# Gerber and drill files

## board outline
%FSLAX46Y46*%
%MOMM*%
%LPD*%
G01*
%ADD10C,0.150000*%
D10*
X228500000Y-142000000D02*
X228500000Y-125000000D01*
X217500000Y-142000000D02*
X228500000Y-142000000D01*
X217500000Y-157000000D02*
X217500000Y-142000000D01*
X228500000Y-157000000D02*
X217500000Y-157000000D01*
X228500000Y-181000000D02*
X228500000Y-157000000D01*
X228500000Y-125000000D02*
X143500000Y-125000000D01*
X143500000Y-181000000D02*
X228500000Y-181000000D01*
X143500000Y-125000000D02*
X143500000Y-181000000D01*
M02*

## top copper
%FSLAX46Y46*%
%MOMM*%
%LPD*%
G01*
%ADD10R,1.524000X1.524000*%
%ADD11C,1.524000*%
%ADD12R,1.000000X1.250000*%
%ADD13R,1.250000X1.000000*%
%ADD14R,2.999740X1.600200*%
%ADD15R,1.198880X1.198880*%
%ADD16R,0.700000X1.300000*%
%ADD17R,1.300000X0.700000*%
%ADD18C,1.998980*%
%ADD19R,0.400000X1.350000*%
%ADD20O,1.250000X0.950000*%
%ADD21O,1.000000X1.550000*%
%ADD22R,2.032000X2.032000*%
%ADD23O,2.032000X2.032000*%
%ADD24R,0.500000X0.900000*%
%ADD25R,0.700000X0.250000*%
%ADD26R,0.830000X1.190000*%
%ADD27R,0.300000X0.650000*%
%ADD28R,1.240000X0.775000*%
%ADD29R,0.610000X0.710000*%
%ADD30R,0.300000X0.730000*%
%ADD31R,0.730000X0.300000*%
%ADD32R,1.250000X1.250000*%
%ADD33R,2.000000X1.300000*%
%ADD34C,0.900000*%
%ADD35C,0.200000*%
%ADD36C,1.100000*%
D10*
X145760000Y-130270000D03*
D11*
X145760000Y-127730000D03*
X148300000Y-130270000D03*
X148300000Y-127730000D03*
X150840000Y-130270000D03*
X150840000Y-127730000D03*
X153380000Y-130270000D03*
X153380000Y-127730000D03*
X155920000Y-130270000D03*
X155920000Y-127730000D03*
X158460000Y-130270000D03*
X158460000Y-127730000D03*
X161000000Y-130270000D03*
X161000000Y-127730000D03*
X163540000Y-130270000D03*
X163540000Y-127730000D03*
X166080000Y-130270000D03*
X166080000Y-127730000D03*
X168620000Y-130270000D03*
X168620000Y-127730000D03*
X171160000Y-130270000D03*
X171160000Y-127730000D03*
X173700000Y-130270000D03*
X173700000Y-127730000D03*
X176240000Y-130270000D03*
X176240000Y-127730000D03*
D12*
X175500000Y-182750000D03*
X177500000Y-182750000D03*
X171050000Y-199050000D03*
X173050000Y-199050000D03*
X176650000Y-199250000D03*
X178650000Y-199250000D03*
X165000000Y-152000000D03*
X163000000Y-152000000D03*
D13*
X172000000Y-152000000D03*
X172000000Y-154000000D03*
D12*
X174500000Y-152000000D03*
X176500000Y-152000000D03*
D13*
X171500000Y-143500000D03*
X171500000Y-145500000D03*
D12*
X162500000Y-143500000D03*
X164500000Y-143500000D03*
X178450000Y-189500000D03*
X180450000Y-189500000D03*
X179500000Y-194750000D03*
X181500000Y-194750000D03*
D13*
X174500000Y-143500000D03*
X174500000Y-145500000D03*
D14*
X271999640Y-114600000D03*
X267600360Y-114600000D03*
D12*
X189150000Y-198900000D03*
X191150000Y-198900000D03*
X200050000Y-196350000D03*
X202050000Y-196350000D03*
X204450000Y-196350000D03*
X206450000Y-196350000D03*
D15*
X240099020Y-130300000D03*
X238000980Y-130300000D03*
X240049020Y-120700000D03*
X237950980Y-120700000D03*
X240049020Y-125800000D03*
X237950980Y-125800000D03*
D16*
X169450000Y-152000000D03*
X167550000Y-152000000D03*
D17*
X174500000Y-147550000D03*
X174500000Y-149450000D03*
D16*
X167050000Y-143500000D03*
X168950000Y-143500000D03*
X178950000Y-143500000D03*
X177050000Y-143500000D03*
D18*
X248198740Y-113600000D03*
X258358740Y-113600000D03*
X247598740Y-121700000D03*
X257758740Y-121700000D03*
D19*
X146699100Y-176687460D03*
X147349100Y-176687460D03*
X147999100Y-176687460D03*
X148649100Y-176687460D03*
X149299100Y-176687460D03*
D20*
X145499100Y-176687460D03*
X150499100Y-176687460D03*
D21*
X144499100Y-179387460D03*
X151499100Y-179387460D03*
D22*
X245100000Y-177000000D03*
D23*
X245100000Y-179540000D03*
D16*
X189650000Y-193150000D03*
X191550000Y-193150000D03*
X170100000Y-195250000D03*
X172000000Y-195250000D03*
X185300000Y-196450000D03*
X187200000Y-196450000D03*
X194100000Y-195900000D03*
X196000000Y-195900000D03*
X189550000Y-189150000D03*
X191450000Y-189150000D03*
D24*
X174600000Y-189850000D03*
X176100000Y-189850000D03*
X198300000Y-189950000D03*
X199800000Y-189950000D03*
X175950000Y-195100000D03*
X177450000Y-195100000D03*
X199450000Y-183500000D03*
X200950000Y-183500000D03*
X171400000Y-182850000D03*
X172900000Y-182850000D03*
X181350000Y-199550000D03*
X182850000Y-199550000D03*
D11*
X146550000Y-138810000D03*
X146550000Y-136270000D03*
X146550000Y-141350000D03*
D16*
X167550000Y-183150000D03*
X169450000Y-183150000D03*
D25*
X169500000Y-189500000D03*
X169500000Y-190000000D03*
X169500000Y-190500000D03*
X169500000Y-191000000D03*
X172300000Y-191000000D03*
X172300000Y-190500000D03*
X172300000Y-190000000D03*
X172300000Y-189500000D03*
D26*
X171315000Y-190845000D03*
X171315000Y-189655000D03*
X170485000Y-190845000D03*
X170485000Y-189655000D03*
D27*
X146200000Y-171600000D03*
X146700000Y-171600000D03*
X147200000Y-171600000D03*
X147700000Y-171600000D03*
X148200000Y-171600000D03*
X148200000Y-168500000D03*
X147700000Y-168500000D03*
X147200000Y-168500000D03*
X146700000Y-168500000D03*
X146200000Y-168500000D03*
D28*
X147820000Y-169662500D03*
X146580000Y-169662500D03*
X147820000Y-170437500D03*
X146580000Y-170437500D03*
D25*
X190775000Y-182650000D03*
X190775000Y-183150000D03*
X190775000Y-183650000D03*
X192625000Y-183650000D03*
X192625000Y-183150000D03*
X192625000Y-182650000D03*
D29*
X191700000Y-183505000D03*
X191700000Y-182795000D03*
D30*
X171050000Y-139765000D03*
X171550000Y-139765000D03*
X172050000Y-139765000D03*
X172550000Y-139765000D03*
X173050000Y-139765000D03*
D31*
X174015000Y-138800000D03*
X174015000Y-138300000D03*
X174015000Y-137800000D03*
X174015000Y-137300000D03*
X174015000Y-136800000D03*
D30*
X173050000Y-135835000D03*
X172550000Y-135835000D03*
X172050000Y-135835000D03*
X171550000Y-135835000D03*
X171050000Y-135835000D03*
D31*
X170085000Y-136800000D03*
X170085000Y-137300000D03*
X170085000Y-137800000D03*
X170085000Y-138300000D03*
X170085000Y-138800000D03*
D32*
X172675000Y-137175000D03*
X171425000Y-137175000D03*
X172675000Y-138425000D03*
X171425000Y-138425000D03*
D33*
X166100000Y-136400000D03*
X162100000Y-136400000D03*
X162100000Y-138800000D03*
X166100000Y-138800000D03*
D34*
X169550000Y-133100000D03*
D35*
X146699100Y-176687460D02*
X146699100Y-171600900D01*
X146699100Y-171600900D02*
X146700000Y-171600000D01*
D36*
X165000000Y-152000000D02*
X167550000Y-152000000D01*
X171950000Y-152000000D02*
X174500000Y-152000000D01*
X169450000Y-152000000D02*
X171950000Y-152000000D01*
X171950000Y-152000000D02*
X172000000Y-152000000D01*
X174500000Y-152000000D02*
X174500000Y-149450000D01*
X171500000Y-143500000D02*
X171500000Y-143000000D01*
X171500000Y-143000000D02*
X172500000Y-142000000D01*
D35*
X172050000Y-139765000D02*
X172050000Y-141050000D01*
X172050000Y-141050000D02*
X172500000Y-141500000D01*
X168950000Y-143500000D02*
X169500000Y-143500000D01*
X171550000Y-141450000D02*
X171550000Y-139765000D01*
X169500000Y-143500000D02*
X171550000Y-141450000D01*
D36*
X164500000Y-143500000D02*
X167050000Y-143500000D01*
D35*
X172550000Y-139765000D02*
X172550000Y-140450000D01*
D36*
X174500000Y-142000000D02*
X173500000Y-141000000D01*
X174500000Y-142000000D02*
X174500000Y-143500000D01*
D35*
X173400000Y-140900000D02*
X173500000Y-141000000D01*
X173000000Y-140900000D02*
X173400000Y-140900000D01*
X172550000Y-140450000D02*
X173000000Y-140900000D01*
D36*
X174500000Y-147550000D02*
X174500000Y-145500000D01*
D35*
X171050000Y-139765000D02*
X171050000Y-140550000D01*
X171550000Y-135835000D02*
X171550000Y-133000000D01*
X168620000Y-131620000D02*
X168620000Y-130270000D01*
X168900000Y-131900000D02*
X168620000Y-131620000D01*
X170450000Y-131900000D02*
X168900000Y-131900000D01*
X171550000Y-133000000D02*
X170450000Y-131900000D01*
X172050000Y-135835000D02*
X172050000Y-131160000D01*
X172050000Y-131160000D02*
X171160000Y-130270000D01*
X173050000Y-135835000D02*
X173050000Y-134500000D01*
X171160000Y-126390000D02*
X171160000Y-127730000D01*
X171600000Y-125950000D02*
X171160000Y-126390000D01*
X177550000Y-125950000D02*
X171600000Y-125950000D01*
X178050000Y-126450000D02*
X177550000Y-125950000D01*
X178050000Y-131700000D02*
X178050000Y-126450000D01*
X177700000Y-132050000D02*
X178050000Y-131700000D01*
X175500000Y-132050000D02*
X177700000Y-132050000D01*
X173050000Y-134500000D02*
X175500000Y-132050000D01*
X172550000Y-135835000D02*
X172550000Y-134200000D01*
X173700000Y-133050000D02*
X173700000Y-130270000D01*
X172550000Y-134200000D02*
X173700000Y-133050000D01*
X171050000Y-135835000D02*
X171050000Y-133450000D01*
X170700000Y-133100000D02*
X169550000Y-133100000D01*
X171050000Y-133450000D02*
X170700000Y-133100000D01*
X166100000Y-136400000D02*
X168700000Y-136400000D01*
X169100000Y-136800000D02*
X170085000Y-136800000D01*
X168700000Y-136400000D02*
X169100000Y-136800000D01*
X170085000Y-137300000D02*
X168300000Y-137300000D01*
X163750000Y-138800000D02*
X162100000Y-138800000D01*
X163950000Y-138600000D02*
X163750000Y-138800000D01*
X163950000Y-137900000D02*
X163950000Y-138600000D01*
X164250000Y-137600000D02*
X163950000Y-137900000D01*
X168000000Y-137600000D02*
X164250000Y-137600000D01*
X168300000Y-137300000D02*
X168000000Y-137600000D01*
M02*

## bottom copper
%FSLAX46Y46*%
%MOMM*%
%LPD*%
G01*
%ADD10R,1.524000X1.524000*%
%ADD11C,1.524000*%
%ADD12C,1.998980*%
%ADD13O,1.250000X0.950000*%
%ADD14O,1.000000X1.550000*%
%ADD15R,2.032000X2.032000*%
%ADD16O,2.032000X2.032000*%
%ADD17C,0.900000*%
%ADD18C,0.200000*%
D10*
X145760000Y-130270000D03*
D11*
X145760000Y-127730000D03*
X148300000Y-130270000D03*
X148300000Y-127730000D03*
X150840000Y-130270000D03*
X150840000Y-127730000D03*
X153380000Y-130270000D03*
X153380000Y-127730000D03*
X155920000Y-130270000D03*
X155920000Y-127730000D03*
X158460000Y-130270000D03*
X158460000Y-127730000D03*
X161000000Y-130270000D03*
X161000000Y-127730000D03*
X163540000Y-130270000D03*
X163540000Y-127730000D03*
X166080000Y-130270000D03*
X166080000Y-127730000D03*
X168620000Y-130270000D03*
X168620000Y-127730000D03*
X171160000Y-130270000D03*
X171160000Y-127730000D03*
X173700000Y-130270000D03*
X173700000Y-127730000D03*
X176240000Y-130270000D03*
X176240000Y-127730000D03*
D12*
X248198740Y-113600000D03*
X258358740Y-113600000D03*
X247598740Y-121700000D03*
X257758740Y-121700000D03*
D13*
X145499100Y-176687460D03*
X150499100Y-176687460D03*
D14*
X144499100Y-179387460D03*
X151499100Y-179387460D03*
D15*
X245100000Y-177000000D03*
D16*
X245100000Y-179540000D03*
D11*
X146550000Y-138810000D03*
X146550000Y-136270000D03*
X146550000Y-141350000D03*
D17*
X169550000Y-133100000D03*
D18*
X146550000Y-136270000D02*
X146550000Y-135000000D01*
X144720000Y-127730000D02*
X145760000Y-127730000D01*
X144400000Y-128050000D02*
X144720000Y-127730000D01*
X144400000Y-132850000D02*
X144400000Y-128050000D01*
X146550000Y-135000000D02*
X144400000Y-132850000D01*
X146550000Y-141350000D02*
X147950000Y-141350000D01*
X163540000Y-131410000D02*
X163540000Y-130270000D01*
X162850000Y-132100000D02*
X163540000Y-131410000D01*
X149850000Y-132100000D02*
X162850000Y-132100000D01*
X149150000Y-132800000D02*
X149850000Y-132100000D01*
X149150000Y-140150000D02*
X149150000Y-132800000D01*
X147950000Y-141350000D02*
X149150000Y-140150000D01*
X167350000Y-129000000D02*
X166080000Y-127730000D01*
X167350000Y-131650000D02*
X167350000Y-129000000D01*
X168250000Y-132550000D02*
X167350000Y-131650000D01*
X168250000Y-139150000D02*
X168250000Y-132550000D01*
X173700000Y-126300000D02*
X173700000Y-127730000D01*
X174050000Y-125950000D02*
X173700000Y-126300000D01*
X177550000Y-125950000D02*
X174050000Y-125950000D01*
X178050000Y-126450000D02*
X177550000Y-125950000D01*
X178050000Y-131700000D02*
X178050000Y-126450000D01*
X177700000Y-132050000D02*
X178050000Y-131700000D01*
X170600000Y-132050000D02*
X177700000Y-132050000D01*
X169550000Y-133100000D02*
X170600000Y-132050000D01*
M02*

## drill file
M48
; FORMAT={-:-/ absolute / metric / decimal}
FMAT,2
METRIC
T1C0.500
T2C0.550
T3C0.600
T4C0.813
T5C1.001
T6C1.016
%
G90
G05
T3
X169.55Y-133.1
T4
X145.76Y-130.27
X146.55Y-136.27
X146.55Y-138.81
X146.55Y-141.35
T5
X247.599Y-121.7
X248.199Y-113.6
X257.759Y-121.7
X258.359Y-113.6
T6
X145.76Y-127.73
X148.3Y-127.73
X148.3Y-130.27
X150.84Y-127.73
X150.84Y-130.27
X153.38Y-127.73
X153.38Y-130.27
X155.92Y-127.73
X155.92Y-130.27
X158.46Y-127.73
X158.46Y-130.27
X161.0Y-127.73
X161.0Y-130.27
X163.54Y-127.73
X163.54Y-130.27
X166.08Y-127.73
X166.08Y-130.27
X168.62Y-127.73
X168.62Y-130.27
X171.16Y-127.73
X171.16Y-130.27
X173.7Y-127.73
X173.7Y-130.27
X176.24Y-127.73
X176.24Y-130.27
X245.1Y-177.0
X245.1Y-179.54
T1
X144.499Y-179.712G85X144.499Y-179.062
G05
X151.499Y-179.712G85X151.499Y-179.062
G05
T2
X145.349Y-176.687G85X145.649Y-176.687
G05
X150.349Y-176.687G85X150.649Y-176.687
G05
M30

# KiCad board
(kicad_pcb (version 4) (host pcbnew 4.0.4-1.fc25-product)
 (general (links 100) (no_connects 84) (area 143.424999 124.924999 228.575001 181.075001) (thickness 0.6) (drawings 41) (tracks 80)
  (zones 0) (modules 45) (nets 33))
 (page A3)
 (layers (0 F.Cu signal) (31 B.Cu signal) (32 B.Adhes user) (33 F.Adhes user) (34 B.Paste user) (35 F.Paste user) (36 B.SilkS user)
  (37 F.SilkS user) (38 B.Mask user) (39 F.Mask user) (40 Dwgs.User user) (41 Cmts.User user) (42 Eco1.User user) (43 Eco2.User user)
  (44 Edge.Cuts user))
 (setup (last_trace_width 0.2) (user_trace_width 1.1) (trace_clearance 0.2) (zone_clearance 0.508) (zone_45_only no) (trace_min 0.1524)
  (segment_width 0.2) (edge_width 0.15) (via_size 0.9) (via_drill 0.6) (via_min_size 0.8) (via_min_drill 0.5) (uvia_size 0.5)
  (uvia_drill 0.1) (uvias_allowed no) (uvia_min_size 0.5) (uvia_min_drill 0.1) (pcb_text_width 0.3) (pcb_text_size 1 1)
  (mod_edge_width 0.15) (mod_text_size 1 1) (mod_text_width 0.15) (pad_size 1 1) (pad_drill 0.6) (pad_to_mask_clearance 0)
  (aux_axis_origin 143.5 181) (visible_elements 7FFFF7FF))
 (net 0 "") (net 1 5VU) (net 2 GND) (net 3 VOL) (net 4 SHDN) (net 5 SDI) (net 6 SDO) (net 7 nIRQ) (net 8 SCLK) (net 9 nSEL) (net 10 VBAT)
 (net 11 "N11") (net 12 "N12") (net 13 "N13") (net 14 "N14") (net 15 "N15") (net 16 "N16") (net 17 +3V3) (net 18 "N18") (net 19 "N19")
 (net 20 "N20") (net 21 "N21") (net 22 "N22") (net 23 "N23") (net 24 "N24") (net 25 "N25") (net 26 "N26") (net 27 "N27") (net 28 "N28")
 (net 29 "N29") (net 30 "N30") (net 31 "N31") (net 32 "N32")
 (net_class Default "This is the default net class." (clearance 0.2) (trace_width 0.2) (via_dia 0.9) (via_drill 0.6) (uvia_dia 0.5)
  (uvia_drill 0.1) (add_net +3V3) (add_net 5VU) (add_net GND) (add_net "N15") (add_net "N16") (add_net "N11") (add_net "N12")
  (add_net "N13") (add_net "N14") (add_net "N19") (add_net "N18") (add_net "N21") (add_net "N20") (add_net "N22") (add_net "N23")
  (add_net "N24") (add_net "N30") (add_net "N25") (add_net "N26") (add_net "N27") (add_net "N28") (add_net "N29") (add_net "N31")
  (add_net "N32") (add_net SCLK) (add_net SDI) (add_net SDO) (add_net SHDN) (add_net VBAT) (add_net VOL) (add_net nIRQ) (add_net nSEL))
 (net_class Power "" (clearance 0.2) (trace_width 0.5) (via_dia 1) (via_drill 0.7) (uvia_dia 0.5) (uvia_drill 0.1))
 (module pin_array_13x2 (layer F.Cu) (at 161 129)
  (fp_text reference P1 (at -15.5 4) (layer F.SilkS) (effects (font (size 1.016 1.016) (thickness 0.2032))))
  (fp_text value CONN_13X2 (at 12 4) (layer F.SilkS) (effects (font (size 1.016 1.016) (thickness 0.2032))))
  (pad 1 thru_hole rect (at -15.24 1.27) (size 1.524 1.524) (drill 0.8128) (layers *.Cu *.Mask F.SilkS))
  (pad 2 thru_hole circle (at -15.24 -1.27) (size 1.524 1.524) (drill 1.016) (layers *.Cu *.Mask F.SilkS) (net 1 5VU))
  (pad 3 thru_hole circle (at -12.7 1.27) (size 1.524 1.524) (drill 1.016) (layers *.Cu *.Mask F.SilkS))
  (pad 4 thru_hole circle (at -12.7 -1.27) (size 1.524 1.524) (drill 1.016) (layers *.Cu *.Mask F.SilkS))
  (pad 5 thru_hole circle (at -10.16 1.27) (size 1.524 1.524) (drill 1.016) (layers *.Cu *.Mask F.SilkS))
  (pad 6 thru_hole circle (at -10.16 -1.27) (size 1.524 1.524) (drill 1.016) (layers *.Cu *.Mask F.SilkS) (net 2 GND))
  (pad 7 thru_hole circle (at -7.62 1.27) (size 1.524 1.524) (drill 1.016) (layers *.Cu *.Mask F.SilkS))
  (pad 8 thru_hole circle (at -7.62 -1.27) (size 1.524 1.524) (drill 1.016) (layers *.Cu *.Mask F.SilkS))
  (pad 9 thru_hole circle (at -5.08 1.27) (size 1.524 1.524) (drill 1.016) (layers *.Cu *.Mask F.SilkS))
  (pad 10 thru_hole circle (at -5.08 -1.27) (size 1.524 1.524) (drill 1.016) (layers *.Cu *.Mask F.SilkS))
  (pad 11 thru_hole circle (at -2.54 1.27) (size 1.524 1.524) (drill 1.016) (layers *.Cu *.Mask F.SilkS))
  (pad 12 thru_hole circle (at -2.54 -1.27) (size 1.524 1.524) (drill 1.016) (layers *.Cu *.Mask F.SilkS))
  (pad 13 thru_hole circle (at 0 1.27) (size 1.524 1.524) (drill 1.016) (layers *.Cu *.Mask F.SilkS))
  (pad 14 thru_hole circle (at 0 -1.27) (size 1.524 1.524) (drill 1.016) (layers *.Cu *.Mask F.SilkS))
  (pad 15 thru_hole circle (at 2.54 1.27) (size 1.524 1.524) (drill 1.016) (layers *.Cu *.Mask F.SilkS) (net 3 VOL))
  (pad 16 thru_hole circle (at 2.54 -1.27) (size 1.524 1.524) (drill 1.016) (layers *.Cu *.Mask F.SilkS))
  (pad 17 thru_hole circle (at 5.08 1.27) (size 1.524 1.524) (drill 1.016) (layers *.Cu *.Mask F.SilkS))
  (pad 18 thru_hole circle (at 5.08 -1.27) (size 1.524 1.524) (drill 1.016) (layers *.Cu *.Mask F.SilkS) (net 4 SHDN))
  (pad 19 thru_hole circle (at 7.62 1.27) (size 1.524 1.524) (drill 1.016) (layers *.Cu *.Mask F.SilkS) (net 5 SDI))
  (pad 20 thru_hole circle (at 7.62 -1.27) (size 1.524 1.524) (drill 1.016) (layers *.Cu *.Mask F.SilkS))
  (pad 21 thru_hole circle (at 10.16 1.27) (size 1.524 1.524) (drill 1.016) (layers *.Cu *.Mask F.SilkS) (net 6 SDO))
  (pad 22 thru_hole circle (at 10.16 -1.27) (size 1.524 1.524) (drill 1.016) (layers *.Cu *.Mask F.SilkS) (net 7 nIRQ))
  (pad 23 thru_hole circle (at 12.7 1.27) (size 1.524 1.524) (drill 1.016) (layers *.Cu *.Mask F.SilkS) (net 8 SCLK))
  (pad 24 thru_hole circle (at 12.7 -1.27) (size 1.524 1.524) (drill 1.016) (layers *.Cu *.Mask F.SilkS) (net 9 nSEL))
  (pad 25 thru_hole circle (at 15.24 1.27) (size 1.524 1.524) (drill 1.016) (layers *.Cu *.Mask F.SilkS))
  (pad 26 thru_hole circle (at 15.24 -1.27) (size 1.524 1.524) (drill 1.016) (layers *.Cu *.Mask F.SilkS)))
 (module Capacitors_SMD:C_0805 (layer F.Cu) (at 176.5 182.75)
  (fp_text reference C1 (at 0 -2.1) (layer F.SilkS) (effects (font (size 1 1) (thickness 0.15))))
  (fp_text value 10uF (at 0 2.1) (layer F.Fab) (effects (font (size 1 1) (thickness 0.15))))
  (pad 1 smd rect (at -1 0) (size 1 1.25) (layers F.Cu F.Paste F.Mask) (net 1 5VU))
  (pad 2 smd rect (at 1 0) (size 1 1.25) (layers F.Cu F.Paste F.Mask) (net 2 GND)))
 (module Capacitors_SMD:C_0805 (layer F.Cu) (at 172.05 199.05)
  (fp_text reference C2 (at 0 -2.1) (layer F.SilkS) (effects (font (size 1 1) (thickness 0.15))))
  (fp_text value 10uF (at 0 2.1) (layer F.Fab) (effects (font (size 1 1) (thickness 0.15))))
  (pad 1 smd rect (at -1 0) (size 1 1.25) (layers F.Cu F.Paste F.Mask) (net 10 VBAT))
  (pad 2 smd rect (at 1 0) (size 1 1.25) (layers F.Cu F.Paste F.Mask) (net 2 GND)))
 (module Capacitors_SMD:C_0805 (layer F.Cu) (at 177.65 199.25)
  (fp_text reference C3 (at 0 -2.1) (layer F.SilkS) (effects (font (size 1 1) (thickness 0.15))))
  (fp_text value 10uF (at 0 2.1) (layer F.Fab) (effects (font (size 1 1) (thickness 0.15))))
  (pad 1 smd rect (at -1 0) (size 1 1.25) (layers F.Cu F.Paste F.Mask) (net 10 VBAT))
  (pad 2 smd rect (at 1 0) (size 1 1.25) (layers F.Cu F.Paste F.Mask) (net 2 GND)))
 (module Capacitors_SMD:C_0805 (layer F.Cu) (at 164 152 180)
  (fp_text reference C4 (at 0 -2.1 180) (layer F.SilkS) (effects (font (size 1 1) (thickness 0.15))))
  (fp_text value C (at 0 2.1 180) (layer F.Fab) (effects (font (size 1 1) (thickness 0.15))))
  (pad 1 smd rect (at -1 0 180) (size 1 1.25) (layers F.Cu F.Paste F.Mask) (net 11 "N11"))
  (pad 2 smd rect (at 1 0 180) (size 1 1.25) (layers F.Cu F.Paste F.Mask)))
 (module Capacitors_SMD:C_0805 (layer F.Cu) (at 172 153 270)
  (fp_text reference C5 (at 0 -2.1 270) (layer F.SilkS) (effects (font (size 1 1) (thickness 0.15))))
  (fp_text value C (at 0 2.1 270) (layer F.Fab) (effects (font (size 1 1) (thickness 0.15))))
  (pad 1 smd rect (at -1 0 270) (size 1 1.25) (layers F.Cu F.Paste F.Mask) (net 11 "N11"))
  (pad 2 smd rect (at 1 0 270) (size 1 1.25) (layers F.Cu F.Paste F.Mask) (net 2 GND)))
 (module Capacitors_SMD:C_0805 (layer F.Cu) (at 175.5 152)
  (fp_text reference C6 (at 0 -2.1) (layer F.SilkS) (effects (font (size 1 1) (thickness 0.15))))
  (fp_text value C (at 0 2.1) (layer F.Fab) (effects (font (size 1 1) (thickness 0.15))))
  (pad 1 smd rect (at -1 0) (size 1 1.25) (layers F.Cu F.Paste F.Mask) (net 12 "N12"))
  (pad 2 smd rect (at 1 0) (size 1 1.25) (layers F.Cu F.Paste F.Mask) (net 2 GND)))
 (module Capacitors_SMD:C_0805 (layer F.Cu) (at 171.5 144.5 270)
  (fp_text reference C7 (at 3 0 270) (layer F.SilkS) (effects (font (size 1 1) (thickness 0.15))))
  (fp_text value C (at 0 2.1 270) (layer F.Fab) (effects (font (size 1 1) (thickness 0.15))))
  (pad 1 smd rect (at -1 0 270) (size 1 1.25) (layers F.Cu F.Paste F.Mask) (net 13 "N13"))
  (pad 2 smd rect (at 1 0 270) (size 1 1.25) (layers F.Cu F.Paste F.Mask)))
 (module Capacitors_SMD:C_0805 (layer F.Cu) (at 163.5 143.5)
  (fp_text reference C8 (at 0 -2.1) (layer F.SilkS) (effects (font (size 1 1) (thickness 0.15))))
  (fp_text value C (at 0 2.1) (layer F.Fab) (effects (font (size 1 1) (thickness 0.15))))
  (pad 1 smd rect (at -1 0) (size 1 1.25) (layers F.Cu F.Paste F.Mask) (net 2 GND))
  (pad 2 smd rect (at 1 0) (size 1 1.25) (layers F.Cu F.Paste F.Mask) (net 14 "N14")))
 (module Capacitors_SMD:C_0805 (layer F.Cu) (at 179.45 189.5)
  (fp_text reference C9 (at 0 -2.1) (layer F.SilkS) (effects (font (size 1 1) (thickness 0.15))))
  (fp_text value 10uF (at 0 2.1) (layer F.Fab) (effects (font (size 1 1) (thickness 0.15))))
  (pad 1 smd rect (at -1 0) (size 1 1.25) (layers F.Cu F.Paste F.Mask) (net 1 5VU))
  (pad 2 smd rect (at 1 0) (size 1 1.25) (layers F.Cu F.Paste F.Mask) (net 2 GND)))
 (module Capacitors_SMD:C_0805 (layer F.Cu) (at 180.5 194.75)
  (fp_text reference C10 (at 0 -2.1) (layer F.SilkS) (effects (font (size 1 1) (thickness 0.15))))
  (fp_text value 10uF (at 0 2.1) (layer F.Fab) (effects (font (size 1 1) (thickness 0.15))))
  (pad 1 smd rect (at -1 0) (size 1 1.25) (layers F.Cu F.Paste F.Mask) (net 10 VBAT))
  (pad 2 smd rect (at 1 0) (size 1 1.25) (layers F.Cu F.Paste F.Mask) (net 2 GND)))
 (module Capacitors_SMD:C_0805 (layer F.Cu) (at 174.5 144.5 270)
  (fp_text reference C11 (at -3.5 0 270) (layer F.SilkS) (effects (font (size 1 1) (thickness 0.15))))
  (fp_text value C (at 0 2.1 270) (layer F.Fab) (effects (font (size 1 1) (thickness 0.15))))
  (pad 1 smd rect (at -1 0 270) (size 1 1.25) (layers F.Cu F.Paste F.Mask) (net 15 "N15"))
  (pad 2 smd rect (at 1 0 270) (size 1 1.25) (layers F.Cu F.Paste F.Mask) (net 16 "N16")))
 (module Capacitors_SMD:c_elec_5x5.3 (layer F.Cu) (at 269.8 114.6)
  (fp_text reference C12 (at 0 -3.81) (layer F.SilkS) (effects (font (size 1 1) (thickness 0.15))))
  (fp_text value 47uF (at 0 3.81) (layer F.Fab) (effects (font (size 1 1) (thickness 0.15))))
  (pad 1 smd rect (at 2.19964 0) (size 2.99974 1.6002) (layers F.Cu F.Paste F.Mask) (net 1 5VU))
  (pad 2 smd rect (at -2.19964 0) (size 2.99974 1.6002) (layers F.Cu F.Paste F.Mask) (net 2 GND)))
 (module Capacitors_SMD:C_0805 (layer F.Cu) (at 190.15 198.9)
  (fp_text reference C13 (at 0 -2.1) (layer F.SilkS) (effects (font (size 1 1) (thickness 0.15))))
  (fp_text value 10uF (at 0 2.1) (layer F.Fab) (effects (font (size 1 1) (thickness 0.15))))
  (pad 1 smd rect (at -1 0) (size 1 1.25) (layers F.Cu F.Paste F.Mask) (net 10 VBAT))
  (pad 2 smd rect (at 1 0) (size 1 1.25) (layers F.Cu F.Paste F.Mask) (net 2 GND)))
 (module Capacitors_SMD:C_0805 (layer F.Cu) (at 201.05 196.35)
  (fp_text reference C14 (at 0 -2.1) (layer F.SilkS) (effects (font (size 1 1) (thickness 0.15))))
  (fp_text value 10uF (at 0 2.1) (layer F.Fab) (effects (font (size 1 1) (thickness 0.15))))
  (pad 1 smd rect (at -1 0) (size 1 1.25) (layers F.Cu F.Paste F.Mask) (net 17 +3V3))
  (pad 2 smd rect (at 1 0) (size 1 1.25) (layers F.Cu F.Paste F.Mask) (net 2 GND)))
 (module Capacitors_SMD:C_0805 (layer F.Cu) (at 205.45 196.35)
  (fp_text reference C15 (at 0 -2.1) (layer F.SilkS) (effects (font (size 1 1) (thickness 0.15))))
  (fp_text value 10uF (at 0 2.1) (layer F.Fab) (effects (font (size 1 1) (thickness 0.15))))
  (pad 1 smd rect (at -1 0) (size 1 1.25) (layers F.Cu F.Paste F.Mask) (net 17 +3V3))
  (pad 2 smd rect (at 1 0) (size 1 1.25) (layers F.Cu F.Paste F.Mask) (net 2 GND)))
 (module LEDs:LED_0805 (layer F.Cu) (at 239.05 130.3)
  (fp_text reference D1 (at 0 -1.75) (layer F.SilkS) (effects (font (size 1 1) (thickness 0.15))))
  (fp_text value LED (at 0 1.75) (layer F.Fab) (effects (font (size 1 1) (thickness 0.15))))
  (pad 2 smd rect (at 1.04902 0 180) (size 1.19888 1.19888) (layers F.Cu F.Paste F.Mask) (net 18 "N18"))
  (pad 1 smd rect (at -1.04902 0 180) (size 1.19888 1.19888) (layers F.Cu F.Paste F.Mask) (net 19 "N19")))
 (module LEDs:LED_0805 (layer F.Cu) (at 239 120.7)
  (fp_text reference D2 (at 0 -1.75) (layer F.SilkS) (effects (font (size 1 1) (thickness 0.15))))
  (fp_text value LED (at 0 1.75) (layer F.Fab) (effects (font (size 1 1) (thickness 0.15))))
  (pad 2 smd rect (at 1.04902 0 180) (size 1.19888 1.19888) (layers F.Cu F.Paste F.Mask) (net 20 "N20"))
  (pad 1 smd rect (at -1.04902 0 180) (size 1.19888 1.19888) (layers F.Cu F.Paste F.Mask) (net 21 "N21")))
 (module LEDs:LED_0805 (layer F.Cu) (at 239 125.8)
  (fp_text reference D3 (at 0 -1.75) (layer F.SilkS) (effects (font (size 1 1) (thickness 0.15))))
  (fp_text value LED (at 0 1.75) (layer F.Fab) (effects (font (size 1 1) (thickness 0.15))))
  (pad 2 smd rect (at 1.04902 0 180) (size 1.19888 1.19888) (layers F.Cu F.Paste F.Mask) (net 1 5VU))
  (pad 1 smd rect (at -1.04902 0 180) (size 1.19888 1.19888) (layers F.Cu F.Paste F.Mask) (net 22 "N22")))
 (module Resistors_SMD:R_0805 (layer F.Cu) (at 168.5 152 180)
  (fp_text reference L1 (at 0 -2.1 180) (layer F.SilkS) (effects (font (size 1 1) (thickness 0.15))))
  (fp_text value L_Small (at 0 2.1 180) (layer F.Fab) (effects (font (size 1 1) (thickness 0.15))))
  (pad 1 smd rect (at -0.95 0 180) (size 0.7 1.3) (layers F.Cu F.Paste F.Mask) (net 12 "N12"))
  (pad 2 smd rect (at 0.95 0 180) (size 0.7 1.3) (layers F.Cu F.Paste F.Mask) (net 11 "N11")))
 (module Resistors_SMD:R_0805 (layer F.Cu) (at 174.5 148.5 270)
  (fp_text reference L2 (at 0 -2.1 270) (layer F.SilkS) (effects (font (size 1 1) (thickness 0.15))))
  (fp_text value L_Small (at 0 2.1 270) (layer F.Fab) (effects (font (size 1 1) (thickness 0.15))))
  (pad 1 smd rect (at -0.95 0 270) (size 0.7 1.3) (layers F.Cu F.Paste F.Mask) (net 16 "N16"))
  (pad 2 smd rect (at 0.95 0 270) (size 0.7 1.3) (layers F.Cu F.Paste F.Mask) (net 12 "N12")))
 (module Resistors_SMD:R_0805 (layer F.Cu) (at 168 143.5)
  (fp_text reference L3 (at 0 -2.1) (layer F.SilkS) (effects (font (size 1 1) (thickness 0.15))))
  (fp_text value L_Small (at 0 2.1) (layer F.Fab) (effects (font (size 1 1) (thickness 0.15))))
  (pad 1 smd rect (at -0.95 0) (size 0.7 1.3) (layers F.Cu F.Paste F.Mask) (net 13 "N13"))
  (pad 2 smd rect (at 0.95 0) (size 0.7 1.3) (layers F.Cu F.Paste F.Mask) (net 14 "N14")))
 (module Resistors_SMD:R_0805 (layer F.Cu) (at 178 143.5 180)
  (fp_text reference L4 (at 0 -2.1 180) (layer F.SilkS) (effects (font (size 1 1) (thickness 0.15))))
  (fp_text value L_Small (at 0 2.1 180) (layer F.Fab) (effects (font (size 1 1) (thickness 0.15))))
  (pad 1 smd rect (at -0.95 0 180) (size 0.7 1.3) (layers F.Cu F.Paste F.Mask) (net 17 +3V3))
  (pad 2 smd rect (at 0.95 0 180) (size 0.7 1.3) (layers F.Cu F.Paste F.Mask) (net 15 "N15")))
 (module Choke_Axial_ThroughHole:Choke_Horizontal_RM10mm (layer F.Cu) (at 253.2 113.6)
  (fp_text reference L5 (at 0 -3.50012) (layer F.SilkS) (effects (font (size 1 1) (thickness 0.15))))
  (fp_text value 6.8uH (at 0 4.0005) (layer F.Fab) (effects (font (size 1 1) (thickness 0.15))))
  (pad 1 thru_hole circle (at -5.00126 0) (size 1.99898 1.99898) (drill 1.00076) (layers *.Cu *.Mask F.SilkS) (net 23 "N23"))
  (pad 2 thru_hole circle (at 5.15874 0) (size 1.99898 1.99898) (drill 1.00076) (layers *.Cu *.Mask F.SilkS) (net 1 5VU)))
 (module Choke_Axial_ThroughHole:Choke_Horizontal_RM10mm (layer F.Cu) (at 252.6 121.7)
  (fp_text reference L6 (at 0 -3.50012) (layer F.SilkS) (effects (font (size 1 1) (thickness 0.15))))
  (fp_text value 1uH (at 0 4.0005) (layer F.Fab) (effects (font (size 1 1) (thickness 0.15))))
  (pad 1 thru_hole circle (at -5.00126 0) (size 1.99898 1.99898) (drill 1.00076) (layers *.Cu *.Mask F.SilkS) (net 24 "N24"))
  (pad 2 thru_hole circle (at 5.15874 0) (size 1.99898 1.99898) (drill 1.00076) (layers *.Cu *.Mask F.SilkS) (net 17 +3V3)))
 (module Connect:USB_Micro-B (layer F.Cu) (at 148 178.25)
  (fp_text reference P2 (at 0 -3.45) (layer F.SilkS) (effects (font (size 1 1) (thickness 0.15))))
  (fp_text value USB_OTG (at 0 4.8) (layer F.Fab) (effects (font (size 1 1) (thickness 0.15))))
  (pad 1 smd rect (at -1.3009 -1.56254 90) (size 1.35 0.4) (layers F.Cu F.Paste F.Mask) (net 1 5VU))
  (pad 2 smd rect (at -0.6509 -1.56254 90) (size 1.35 0.4) (layers F.Cu F.Paste F.Mask))
  (pad 3 smd rect (at -0.0009 -1.56254 90) (size 1.35 0.4) (layers F.Cu F.Paste F.Mask))
  (pad 4 smd rect (at 0.6491 -1.56254 90) (size 1.35 0.4) (layers F.Cu F.Paste F.Mask))
  (pad 5 smd rect (at 1.2991 -1.56254 90) (size 1.35 0.4) (layers F.Cu F.Paste F.Mask) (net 2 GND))
  (pad 6 thru_hole oval (at -2.5009 -1.56254 90) (size 0.95 1.25) (drill oval 0.55 0.85) (layers *.Cu *.Mask F.SilkS) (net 2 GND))
  (pad 6 thru_hole oval (at 2.4991 -1.56254 90) (size 0.95 1.25) (drill oval 0.55 0.85) (layers *.Cu *.Mask F.SilkS) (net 2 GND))
  (pad 6 thru_hole oval (at -3.5009 1.13746 90) (size 1.55 1) (drill oval 1.15 0.5) (layers *.Cu *.Mask F.SilkS) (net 2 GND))
  (pad 6 thru_hole oval (at 3.4991 1.13746 90) (size 1.55 1) (drill oval 1.15 0.5) (layers *.Cu *.Mask F.SilkS) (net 2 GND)))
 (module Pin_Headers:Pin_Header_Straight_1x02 (layer F.Cu) (at 245.1 177)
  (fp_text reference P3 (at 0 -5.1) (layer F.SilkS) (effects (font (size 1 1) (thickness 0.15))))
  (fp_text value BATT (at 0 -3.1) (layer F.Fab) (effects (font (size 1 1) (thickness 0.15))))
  (pad 1 thru_hole rect (at 0 0) (size 2.032 2.032) (drill 1.016) (layers *.Cu *.Mask F.SilkS) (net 2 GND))
  (pad 2 thru_hole oval (at 0 2.54) (size 2.032 2.032) (drill 1.016) (layers *.Cu *.Mask F.SilkS)))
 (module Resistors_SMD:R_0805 (layer F.Cu) (at 190.6 193.15)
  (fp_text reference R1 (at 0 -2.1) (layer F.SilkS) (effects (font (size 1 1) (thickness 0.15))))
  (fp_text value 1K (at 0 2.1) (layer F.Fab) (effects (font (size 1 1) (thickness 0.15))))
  (pad 1 smd rect (at -0.95 0) (size 0.7 1.3) (layers F.Cu F.Paste F.Mask) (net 1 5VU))
  (pad 2 smd rect (at 0.95 0) (size 0.7 1.3) (layers F.Cu F.Paste F.Mask) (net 18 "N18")))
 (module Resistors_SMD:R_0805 (layer F.Cu) (at 171.05 195.25)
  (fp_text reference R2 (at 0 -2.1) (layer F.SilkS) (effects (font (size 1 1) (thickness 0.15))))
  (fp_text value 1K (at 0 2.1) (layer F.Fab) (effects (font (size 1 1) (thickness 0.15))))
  (pad 1 smd rect (at -0.95 0) (size 0.7 1.3) (layers F.Cu F.Paste F.Mask) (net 1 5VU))
  (pad 2 smd rect (at 0.95 0) (size 0.7 1.3) (layers F.Cu F.Paste F.Mask) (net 20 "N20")))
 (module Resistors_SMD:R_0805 (layer F.Cu) (at 186.25 196.45)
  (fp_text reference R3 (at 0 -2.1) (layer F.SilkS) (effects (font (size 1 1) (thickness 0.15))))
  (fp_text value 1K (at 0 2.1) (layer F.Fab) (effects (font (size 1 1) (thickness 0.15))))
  (pad 1 smd rect (at -0.95 0) (size 0.7 1.3) (layers F.Cu F.Paste F.Mask) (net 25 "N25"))
  (pad 2 smd rect (at 0.95 0) (size 0.7 1.3) (layers F.Cu F.Paste F.Mask) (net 2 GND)))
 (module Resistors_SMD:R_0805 (layer F.Cu) (at 195.05 195.9)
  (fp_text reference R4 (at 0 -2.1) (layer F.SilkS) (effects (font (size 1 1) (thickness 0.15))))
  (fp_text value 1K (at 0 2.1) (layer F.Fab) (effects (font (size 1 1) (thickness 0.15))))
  (pad 1 smd rect (at -0.95 0) (size 0.7 1.3) (layers F.Cu F.Paste F.Mask) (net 22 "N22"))
  (pad 2 smd rect (at 0.95 0) (size 0.7 1.3) (layers F.Cu F.Paste F.Mask) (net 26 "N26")))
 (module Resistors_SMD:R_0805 (layer F.Cu) (at 190.5 189.15)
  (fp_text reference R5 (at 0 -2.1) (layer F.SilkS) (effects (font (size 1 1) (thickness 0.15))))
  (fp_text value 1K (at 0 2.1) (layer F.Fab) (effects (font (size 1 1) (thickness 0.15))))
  (pad 1 smd rect (at -0.95 0) (size 0.7 1.3) (layers F.Cu F.Paste F.Mask) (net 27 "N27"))
  (pad 2 smd rect (at 0.95 0) (size 0.7 1.3) (layers F.Cu F.Paste F.Mask)))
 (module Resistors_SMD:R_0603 (layer F.Cu) (at 175.35 189.85)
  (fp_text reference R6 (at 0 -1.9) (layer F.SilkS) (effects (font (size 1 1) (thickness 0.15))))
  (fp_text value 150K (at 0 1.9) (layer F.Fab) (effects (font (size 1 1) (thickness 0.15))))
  (pad 1 smd rect (at -0.75 0) (size 0.5 0.9) (layers F.Cu F.Paste F.Mask) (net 27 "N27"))
  (pad 2 smd rect (at 0.75 0) (size 0.5 0.9) (layers F.Cu F.Paste F.Mask) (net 2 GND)))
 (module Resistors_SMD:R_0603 (layer F.Cu) (at 199.05 189.95)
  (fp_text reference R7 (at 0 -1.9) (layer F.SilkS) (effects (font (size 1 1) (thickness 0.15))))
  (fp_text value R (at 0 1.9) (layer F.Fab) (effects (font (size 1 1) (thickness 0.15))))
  (pad 1 smd rect (at -0.75 0) (size 0.5 0.9) (layers F.Cu F.Paste F.Mask) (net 1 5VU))
  (pad 2 smd rect (at 0.75 0) (size 0.5 0.9) (layers F.Cu F.Paste F.Mask) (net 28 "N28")))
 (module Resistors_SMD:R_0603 (layer F.Cu) (at 176.7 195.1)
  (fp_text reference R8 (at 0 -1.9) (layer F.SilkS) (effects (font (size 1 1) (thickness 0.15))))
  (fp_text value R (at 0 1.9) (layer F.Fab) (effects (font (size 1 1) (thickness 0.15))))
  (pad 1 smd rect (at -0.75 0) (size 0.5 0.9) (layers F.Cu F.Paste F.Mask) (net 28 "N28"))
  (pad 2 smd rect (at 0.75 0) (size 0.5 0.9) (layers F.Cu F.Paste F.Mask) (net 2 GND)))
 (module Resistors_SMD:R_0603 (layer F.Cu) (at 200.2 183.5)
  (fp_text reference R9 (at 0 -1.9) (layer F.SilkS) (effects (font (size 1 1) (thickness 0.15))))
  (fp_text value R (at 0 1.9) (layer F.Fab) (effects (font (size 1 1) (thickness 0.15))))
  (pad 1 smd rect (at -0.75 0) (size 0.5 0.9) (layers F.Cu F.Paste F.Mask) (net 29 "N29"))
  (pad 2 smd rect (at 0.75 0) (size 0.5 0.9) (layers F.Cu F.Paste F.Mask) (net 1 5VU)))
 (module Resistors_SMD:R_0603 (layer F.Cu) (at 172.15 182.85)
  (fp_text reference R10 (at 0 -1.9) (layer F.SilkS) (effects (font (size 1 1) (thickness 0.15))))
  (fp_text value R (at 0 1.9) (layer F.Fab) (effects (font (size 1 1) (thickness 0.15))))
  (pad 1 smd rect (at -0.75 0) (size 0.5 0.9) (layers F.Cu F.Paste F.Mask) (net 10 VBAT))
  (pad 2 smd rect (at 0.75 0) (size 0.5 0.9) (layers F.Cu F.Paste F.Mask) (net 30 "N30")))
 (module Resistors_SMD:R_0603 (layer F.Cu) (at 182.1 199.55)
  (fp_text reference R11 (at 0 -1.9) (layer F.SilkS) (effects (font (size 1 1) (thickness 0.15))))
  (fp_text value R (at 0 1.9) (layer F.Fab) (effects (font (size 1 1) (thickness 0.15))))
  (pad 1 smd rect (at -0.75 0) (size 0.5 0.9) (layers F.Cu F.Paste F.Mask) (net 30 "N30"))
  (pad 2 smd rect (at 0.75 0) (size 0.5 0.9) (layers F.Cu F.Paste F.Mask) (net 2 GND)))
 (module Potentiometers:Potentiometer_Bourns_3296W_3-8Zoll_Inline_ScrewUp (layer F.Cu) (at 146.55 141.35)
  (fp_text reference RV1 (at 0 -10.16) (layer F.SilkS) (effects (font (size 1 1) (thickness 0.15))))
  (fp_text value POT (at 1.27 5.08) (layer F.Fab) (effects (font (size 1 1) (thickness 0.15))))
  (pad 2 thru_hole circle (at 0 -2.54) (size 1.524 1.524) (drill 0.8128) (layers *.Cu *.Mask F.SilkS) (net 2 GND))
  (pad 3 thru_hole circle (at 0 -5.08) (size 1.524 1.524) (drill 0.8128) (layers *.Cu *.Mask F.SilkS) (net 1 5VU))
  (pad 1 thru_hole circle (at 0 0) (size 1.524 1.524) (drill 0.8128) (layers *.Cu *.Mask F.SilkS) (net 3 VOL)))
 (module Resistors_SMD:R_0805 (layer F.Cu) (at 168.5 183.15)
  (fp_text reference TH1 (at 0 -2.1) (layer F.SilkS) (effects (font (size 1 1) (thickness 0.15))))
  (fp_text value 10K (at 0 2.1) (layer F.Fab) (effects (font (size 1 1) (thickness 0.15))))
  (pad 1 smd rect (at -0.95 0) (size 0.7 1.3) (layers F.Cu F.Paste F.Mask) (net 27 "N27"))
  (pad 2 smd rect (at 0.95 0) (size 0.7 1.3) (layers F.Cu F.Paste F.Mask) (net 2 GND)))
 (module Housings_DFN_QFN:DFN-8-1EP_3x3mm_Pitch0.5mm (layer F.Cu) (at 170.9 190.25)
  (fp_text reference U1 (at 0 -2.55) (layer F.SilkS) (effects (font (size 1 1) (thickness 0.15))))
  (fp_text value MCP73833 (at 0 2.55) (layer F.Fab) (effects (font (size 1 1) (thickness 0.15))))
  (pad 1 smd rect (at -1.4 -0.75) (size 0.7 0.25) (layers F.Cu F.Paste F.Mask) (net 1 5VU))
  (pad 2 smd rect (at -1.4 -0.25) (size 0.7 0.25) (layers F.Cu F.Paste F.Mask) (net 1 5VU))
  (pad 3 smd rect (at -1.4 0.25) (size 0.7 0.25) (layers F.Cu F.Paste F.Mask) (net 21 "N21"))
  (pad 4 smd rect (at -1.4 0.75) (size 0.7 0.25) (layers F.Cu F.Paste F.Mask) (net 19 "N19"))
  (pad 5 smd rect (at 1.4 0.75) (size 0.7 0.25) (layers F.Cu F.Paste F.Mask) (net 2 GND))
  (pad 6 smd rect (at 1.4 0.25) (size 0.7 0.25) (layers F.Cu F.Paste F.Mask) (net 25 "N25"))
  (pad 7 smd rect (at 1.4 -0.25) (size 0.7 0.25) (layers F.Cu F.Paste F.Mask))
  (pad 8 smd rect (at 1.4 -0.75) (size 0.7 0.25) (layers F.Cu F.Paste F.Mask) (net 26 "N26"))
  (pad 9 smd rect (at 0.415 0.595) (size 0.83 1.19) (layers F.Cu F.Paste F.Mask) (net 10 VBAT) (solder_paste_margin_ratio -0.2))
  (pad 9 smd rect (at 0.415 -0.595) (size 0.83 1.19) (layers F.Cu F.Paste F.Mask) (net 10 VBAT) (solder_paste_margin_ratio -0.2))
  (pad 9 smd rect (at -0.415 0.595) (size 0.83 1.19) (layers F.Cu F.Paste F.Mask) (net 10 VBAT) (solder_paste_margin_ratio -0.2))
  (pad 9 smd rect (at -0.415 -0.595) (size 0.83 1.19) (layers F.Cu F.Paste F.Mask) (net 10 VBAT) (solder_paste_margin_ratio -0.2)))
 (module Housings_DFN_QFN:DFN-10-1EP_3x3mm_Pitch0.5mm (layer F.Cu) (at 147.2 170.05 90)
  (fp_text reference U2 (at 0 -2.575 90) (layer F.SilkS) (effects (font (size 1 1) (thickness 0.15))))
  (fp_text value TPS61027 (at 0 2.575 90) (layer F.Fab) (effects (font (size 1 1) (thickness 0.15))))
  (pad 1 smd rect (at -1.55 -1 90) (size 0.65 0.3) (layers F.Cu F.Paste F.Mask) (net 10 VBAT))
  (pad 2 smd rect (at -1.55 -0.5 90) (size 0.65 0.3) (layers F.Cu F.Paste F.Mask) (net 1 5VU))
  (pad 3 smd rect (at -1.55 0 90) (size 0.65 0.3) (layers F.Cu F.Paste F.Mask) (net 28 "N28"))
  (pad 4 smd rect (at -1.55 0.5 90) (size 0.65 0.3) (layers F.Cu F.Paste F.Mask) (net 29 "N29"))
  (pad 5 smd rect (at -1.55 1 90) (size 0.65 0.3) (layers F.Cu F.Paste F.Mask) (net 2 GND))
  (pad 6 smd rect (at 1.55 1 90) (size 0.65 0.3) (layers F.Cu F.Paste F.Mask) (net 10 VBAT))
  (pad 7 smd rect (at 1.55 0.5 90) (size 0.65 0.3) (layers F.Cu F.Paste F.Mask) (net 30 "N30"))
  (pad 8 smd rect (at 1.55 0 90) (size 0.65 0.3) (layers F.Cu F.Paste F.Mask) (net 2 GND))
  (pad 9 smd rect (at 1.55 -0.5 90) (size 0.65 0.3) (layers F.Cu F.Paste F.Mask) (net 23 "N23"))
  (pad 10 smd rect (at 1.55 -1 90) (size 0.65 0.3) (layers F.Cu F.Paste F.Mask) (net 2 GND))
  (pad 11 smd rect (at 0.3875 0.62 90) (size 0.775 1.24) (layers F.Cu F.Paste F.Mask) (solder_paste_margin_ratio -0.2))
  (pad 11 smd rect (at 0.3875 -0.62 90) (size 0.775 1.24) (layers F.Cu F.Paste F.Mask) (solder_paste_margin_ratio -0.2))
  (pad 11 smd rect (at -0.3875 0.62 90) (size 0.775 1.24) (layers F.Cu F.Paste F.Mask) (solder_paste_margin_ratio -0.2))
  (pad 11 smd rect (at -0.3875 -0.62 90) (size 0.775 1.24) (layers F.Cu F.Paste F.Mask) (solder_paste_margin_ratio -0.2)))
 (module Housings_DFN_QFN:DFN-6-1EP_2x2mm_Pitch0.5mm (layer F.Cu) (at 191.7 183.15)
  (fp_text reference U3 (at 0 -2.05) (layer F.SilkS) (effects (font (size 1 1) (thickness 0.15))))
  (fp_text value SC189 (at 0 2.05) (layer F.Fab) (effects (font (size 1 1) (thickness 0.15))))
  (pad 1 smd rect (at -0.925 -0.5) (size 0.7 0.25) (layers F.Cu F.Paste F.Mask) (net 10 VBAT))
  (pad 2 smd rect (at -0.925 0) (size 0.7 0.25) (layers F.Cu F.Paste F.Mask) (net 2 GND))
  (pad 3 smd rect (at -0.925 0.5) (size 0.7 0.25) (layers F.Cu F.Paste F.Mask) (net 10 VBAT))
  (pad 4 smd rect (at 0.925 0.5) (size 0.7 0.25) (layers F.Cu F.Paste F.Mask) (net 17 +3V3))
  (pad 5 smd rect (at 0.925 0) (size 0.7 0.25) (layers F.Cu F.Paste F.Mask) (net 24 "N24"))
  (pad 6 smd rect (at 0.925 -0.5) (size 0.7 0.25) (layers F.Cu F.Paste F.Mask))
  (pad 7 smd rect (at 0 0.355) (size 0.61 0.71) (layers F.Cu F.Paste F.Mask) (solder_paste_margin_ratio -0.2))
  (pad 7 smd rect (at 0 -0.355) (size 0.61 0.71) (layers F.Cu F.Paste F.Mask) (solder_paste_margin_ratio -0.2)))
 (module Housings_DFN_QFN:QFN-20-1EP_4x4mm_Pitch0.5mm (layer F.Cu) (at 172.05 137.8 90)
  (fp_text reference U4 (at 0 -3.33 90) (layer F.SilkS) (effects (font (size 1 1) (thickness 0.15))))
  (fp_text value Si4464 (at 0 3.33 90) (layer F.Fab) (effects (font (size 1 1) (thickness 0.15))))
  (pad 1 smd rect (at -1.965 -1 90) (size 0.73 0.3) (layers F.Cu F.Paste F.Mask) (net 4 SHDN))
  (pad 2 smd rect (at -1.965 -0.5 90) (size 0.73 0.3) (layers F.Cu F.Paste F.Mask) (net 14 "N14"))
  (pad 3 smd rect (at -1.965 0 90) (size 0.73 0.3) (layers F.Cu F.Paste F.Mask) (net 13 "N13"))
  (pad 4 smd rect (at -1.965 0.5 90) (size 0.73 0.3) (layers F.Cu F.Paste F.Mask) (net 15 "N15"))
  (pad 5 smd rect (at -1.965 1 90) (size 0.73 0.3) (layers F.Cu F.Paste F.Mask))
  (pad 6 smd rect (at -1 1.965 180) (size 0.73 0.3) (layers F.Cu F.Paste F.Mask) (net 17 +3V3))
  (pad 7 smd rect (at -0.5 1.965 180) (size 0.73 0.3) (layers F.Cu F.Paste F.Mask))
  (pad 8 smd rect (at 0 1.965 180) (size 0.73 0.3) (layers F.Cu F.Paste F.Mask) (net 17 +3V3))
  (pad 9 smd rect (at 0.5 1.965 180) (size 0.73 0.3) (layers F.Cu F.Paste F.Mask))
  (pad 10 smd rect (at 1 1.965 180) (size 0.73 0.3) (layers F.Cu F.Paste F.Mask))
  (pad 11 smd rect (at 1.965 1 90) (size 0.73 0.3) (layers F.Cu F.Paste F.Mask) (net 7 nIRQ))
  (pad 12 smd rect (at 1.965 0.5 90) (size 0.73 0.3) (layers F.Cu F.Paste F.Mask) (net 8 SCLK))
  (pad 13 smd rect (at 1.965 0 90) (size 0.73 0.3) (layers F.Cu F.Paste F.Mask) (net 6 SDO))
  (pad 14 smd rect (at 1.965 -0.5 90) (size 0.73 0.3) (layers F.Cu F.Paste F.Mask) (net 5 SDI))
  (pad 15 smd rect (at 1.965 -1 90) (size 0.73 0.3) (layers F.Cu F.Paste F.Mask) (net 9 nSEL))
  (pad 16 smd rect (at 1 -1.965 180) (size 0.73 0.3) (layers F.Cu F.Paste F.Mask) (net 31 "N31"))
  (pad 17 smd rect (at 0.5 -1.965 180) (size 0.73 0.3) (layers F.Cu F.Paste F.Mask) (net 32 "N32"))
  (pad 18 smd rect (at 0 -1.965 180) (size 0.73 0.3) (layers F.Cu F.Paste F.Mask) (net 2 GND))
  (pad 19 smd rect (at -0.5 -1.965 180) (size 0.73 0.3) (layers F.Cu F.Paste F.Mask))
  (pad 20 smd rect (at -1 -1.965 180) (size 0.73 0.3) (layers F.Cu F.Paste F.Mask))
  (pad 21 smd rect (at 0.625 0.625 90) (size 1.25 1.25) (layers F.Cu F.Paste F.Mask) (solder_paste_margin_ratio -0.2))
  (pad 21 smd rect (at 0.625 -0.625 90) (size 1.25 1.25) (layers F.Cu F.Paste F.Mask) (solder_paste_margin_ratio -0.2))
  (pad 21 smd rect (at -0.625 0.625 90) (size 1.25 1.25) (layers F.Cu F.Paste F.Mask) (solder_paste_margin_ratio -0.2))
  (pad 21 smd rect (at -0.625 -0.625 90) (size 1.25 1.25) (layers F.Cu F.Paste F.Mask) (solder_paste_margin_ratio -0.2)))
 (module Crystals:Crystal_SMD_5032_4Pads (layer F.Cu) (at 164.1 137.6 180)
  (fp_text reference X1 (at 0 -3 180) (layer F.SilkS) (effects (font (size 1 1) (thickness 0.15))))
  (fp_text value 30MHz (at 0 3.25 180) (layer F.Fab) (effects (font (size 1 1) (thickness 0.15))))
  (pad 1 smd rect (at -2 1.2 180) (size 2 1.3) (layers F.Cu F.Paste F.Mask) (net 31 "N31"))
  (pad 3 smd rect (at 2 1.2 180) (size 2 1.3) (layers F.Cu F.Paste F.Mask) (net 2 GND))
  (pad 2 smd rect (at 2 -1.2 180) (size 2 1.3) (layers F.Cu F.Paste F.Mask) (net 32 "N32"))
  (pad 3 smd rect (at -2 -1.2 180) (size 2 1.3) (layers F.Cu F.Paste F.Mask) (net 2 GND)))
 (gr_line (start 228.5 142) (end 228.5 125) (angle 90) (layer Edge.Cuts) (width 0.15))
 (gr_line (start 217.5 142) (end 228.5 142) (angle 90) (layer Edge.Cuts) (width 0.15))
 (gr_line (start 217.5 157) (end 217.5 142) (angle 90) (layer Edge.Cuts) (width 0.15))
 (gr_line (start 228.5 157) (end 217.5 157) (angle 90) (layer Edge.Cuts) (width 0.15))
 (gr_line (start 228.5 181) (end 228.5 157) (angle 90) (layer Edge.Cuts) (width 0.15))
 (gr_line (start 228.5 125) (end 143.5 125) (angle 90) (layer Edge.Cuts) (width 0.15))
 (gr_line (start 143.5 181) (end 228.5 181) (angle 90) (layer Edge.Cuts) (width 0.15))
 (gr_line (start 143.5 125) (end 143.5 181) (angle 90) (layer Edge.Cuts) (width 0.15))
 (segment (start 146.6991 176.68746) (end 146.6991 171.6009) (width 0.2) (layer F.Cu) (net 1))
 (segment (start 146.6991 171.6009) (end 146.7 171.6) (width 0.2) (layer F.Cu) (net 1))
 (segment (start 146.55 136.27) (end 146.55 135) (width 0.2) (layer B.Cu) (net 1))
 (segment (start 144.72 127.73) (end 145.76 127.73) (width 0.2) (layer B.Cu) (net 1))
 (segment (start 144.4 128.05) (end 144.72 127.73) (width 0.2) (layer B.Cu) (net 1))
 (segment (start 144.4 132.85) (end 144.4 128.05) (width 0.2) (layer B.Cu) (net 1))
 (segment (start 146.55 135) (end 144.4 132.85) (width 0.2) (layer B.Cu) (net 1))
 (segment (start 165 152) (end 167.55 152) (width 1.1) (layer F.Cu) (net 11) (status C00000))
 (segment (start 171.95 152) (end 174.5 152) (width 1.1) (layer F.Cu) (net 11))
 (segment (start 169.45 152) (end 171.95 152) (width 1.1) (layer F.Cu) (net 12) (status C00000))
 (segment (start 171.95 152) (end 172 152) (width 1.1) (layer F.Cu) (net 12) (status C00000))
 (segment (start 174.5 152) (end 174.5 149.45) (width 1.1) (layer F.Cu) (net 12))
 (segment (start 171.5 143.5) (end 171.5 143) (width 1.1) (layer F.Cu) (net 13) (status C00000))
 (segment (start 171.5 143) (end 172.5 142) (width 1.1) (layer F.Cu) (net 13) (status 400000))
 (segment (start 172.05 139.765) (end 172.05 141.05) (width 0.2) (layer F.Cu) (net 13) (status 400000))
 (segment (start 172.05 141.05) (end 172.5 141.5) (width 0.2) (layer F.Cu) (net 13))
 (segment (start 168.95 143.5) (end 169.5 143.5) (width 0.2) (layer F.Cu) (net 14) (status 400000))
 (segment (start 171.55 141.45) (end 171.55 139.765) (width 0.2) (layer F.Cu) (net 14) (status 800000))
 (segment (start 169.5 143.5) (end 171.55 141.45) (width 0.2) (layer F.Cu) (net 14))
 (segment (start 164.5 143.5) (end 167.05 143.5) (width 1.1) (layer F.Cu) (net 14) (status C00000))
 (segment (start 172.55 139.765) (end 172.55 140.45) (width 0.2) (layer F.Cu) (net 15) (status 400000))
 (segment (start 174.5 142) (end 173.5 141) (width 1.1) (layer F.Cu) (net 15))
 (segment (start 174.5 142) (end 174.5 143.5) (width 1.1) (layer F.Cu) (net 15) (status 800000))
 (segment (start 173.4 140.9) (end 173.5 141) (width 0.2) (layer F.Cu) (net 15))
 (segment (start 173 140.9) (end 173.4 140.9) (width 0.2) (layer F.Cu) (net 15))
 (segment (start 172.55 140.45) (end 173 140.9) (width 0.2) (layer F.Cu) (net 15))
 (segment (start 174.5 147.55) (end 174.5 145.5) (width 1.1) (layer F.Cu) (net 16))
 (segment (start 146.55 141.35) (end 147.95 141.35) (width 0.2) (layer B.Cu) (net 3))
 (segment (start 163.54 131.41) (end 163.54 130.27) (width 0.2) (layer B.Cu) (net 3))
 (segment (start 162.85 132.1) (end 163.54 131.41) (width 0.2) (layer B.Cu) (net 3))
 (segment (start 149.85 132.1) (end 162.85 132.1) (width 0.2) (layer B.Cu) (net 3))
 (segment (start 149.15 132.8) (end 149.85 132.1) (width 0.2) (layer B.Cu) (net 3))
 (segment (start 149.15 140.15) (end 149.15 132.8) (width 0.2) (layer B.Cu) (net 3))
 (segment (start 147.95 141.35) (end 149.15 140.15) (width 0.2) (layer B.Cu) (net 3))
 (segment (start 171.05 139.765) (end 171.05 140.55) (width 0.2) (layer F.Cu) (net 4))
 (segment (start 167.35 129) (end 166.08 127.73) (width 0.2) (layer B.Cu) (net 4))
 (segment (start 167.35 131.65) (end 167.35 129) (width 0.2) (layer B.Cu) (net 4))
 (segment (start 168.25 132.55) (end 167.35 131.65) (width 0.2) (layer B.Cu) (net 4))
 (segment (start 168.25 139.15) (end 168.25 132.55) (width 0.2) (layer B.Cu) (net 4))
 (segment (start 171.55 135.835) (end 171.55 133) (width 0.2) (layer F.Cu) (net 5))
 (segment (start 168.62 131.62) (end 168.62 130.27) (width 0.2) (layer F.Cu) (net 5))
 (segment (start 168.9 131.9) (end 168.62 131.62) (width 0.2) (layer F.Cu) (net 5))
 (segment (start 170.45 131.9) (end 168.9 131.9) (width 0.2) (layer F.Cu) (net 5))
 (segment (start 171.55 133) (end 170.45 131.9) (width 0.2) (layer F.Cu) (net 5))
 (segment (start 172.05 135.835) (end 172.05 131.16) (width 0.2) (layer F.Cu) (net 6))
 (segment (start 172.05 131.16) (end 171.16 130.27) (width 0.2) (layer F.Cu) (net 6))
 (segment (start 173.05 135.835) (end 173.05 134.5) (width 0.2) (layer F.Cu) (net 7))
 (segment (start 171.16 126.39) (end 171.16 127.73) (width 0.2) (layer F.Cu) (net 7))
 (segment (start 171.6 125.95) (end 171.16 126.39) (width 0.2) (layer F.Cu) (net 7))
 (segment (start 177.55 125.95) (end 171.6 125.95) (width 0.2) (layer F.Cu) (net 7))
 (segment (start 178.05 126.45) (end 177.55 125.95) (width 0.2) (layer F.Cu) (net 7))
 (segment (start 178.05 131.7) (end 178.05 126.45) (width 0.2) (layer F.Cu) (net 7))
 (segment (start 177.7 132.05) (end 178.05 131.7) (width 0.2) (layer F.Cu) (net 7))
 (segment (start 175.5 132.05) (end 177.7 132.05) (width 0.2) (layer F.Cu) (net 7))
 (segment (start 173.05 134.5) (end 175.5 132.05) (width 0.2) (layer F.Cu) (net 7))
 (segment (start 172.55 135.835) (end 172.55 134.2) (width 0.2) (layer F.Cu) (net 8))
 (segment (start 173.7 133.05) (end 173.7 130.27) (width 0.2) (layer F.Cu) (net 8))
 (segment (start 172.55 134.2) (end 173.7 133.05) (width 0.2) (layer F.Cu) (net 8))
 (segment (start 171.05 135.835) (end 171.05 133.45) (width 0.2) (layer F.Cu) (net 9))
 (segment (start 173.7 126.3) (end 173.7 127.73) (width 0.2) (layer B.Cu) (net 9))
 (segment (start 174.05 125.95) (end 173.7 126.3) (width 0.2) (layer B.Cu) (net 9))
 (segment (start 177.55 125.95) (end 174.05 125.95) (width 0.2) (layer B.Cu) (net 9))
 (segment (start 178.05 126.45) (end 177.55 125.95) (width 0.2) (layer B.Cu) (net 9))
 (segment (start 178.05 131.7) (end 178.05 126.45) (width 0.2) (layer B.Cu) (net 9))
 (segment (start 177.7 132.05) (end 178.05 131.7) (width 0.2) (layer B.Cu) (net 9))
 (segment (start 170.6 132.05) (end 177.7 132.05) (width 0.2) (layer B.Cu) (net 9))
 (segment (start 169.55 133.1) (end 170.6 132.05) (width 0.2) (layer B.Cu) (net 9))
 (via (at 169.55 133.1) (size 0.9) (drill 0.6) (layers F.Cu B.Cu) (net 9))
 (segment (start 170.7 133.1) (end 169.55 133.1) (width 0.2) (layer F.Cu) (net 9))
 (segment (start 171.05 133.45) (end 170.7 133.1) (width 0.2) (layer F.Cu) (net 9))
 (segment (start 166.1 136.4) (end 168.7 136.4) (width 0.2) (layer F.Cu) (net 31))
 (segment (start 169.1 136.8) (end 170.085 136.8) (width 0.2) (layer F.Cu) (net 31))
 (segment (start 168.7 136.4) (end 169.1 136.8) (width 0.2) (layer F.Cu) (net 31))
 (segment (start 170.085 137.3) (end 168.3 137.3) (width 0.2) (layer F.Cu) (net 32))
 (segment (start 163.75 138.8) (end 162.1 138.8) (width 0.2) (layer F.Cu) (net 32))
 (segment (start 163.95 138.6) (end 163.75 138.8) (width 0.2) (layer F.Cu) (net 32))
 (segment (start 163.95 137.9) (end 163.95 138.6) (width 0.2) (layer F.Cu) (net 32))
 (segment (start 164.25 137.6) (end 163.95 137.9) (width 0.2) (layer F.Cu) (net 32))
 (segment (start 168 137.6) (end 164.25 137.6) (width 0.2) (layer F.Cu) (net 32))
 (segment (start 168.3 137.3) (end 168 137.6) (width 0.2) (layer F.Cu) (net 32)))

